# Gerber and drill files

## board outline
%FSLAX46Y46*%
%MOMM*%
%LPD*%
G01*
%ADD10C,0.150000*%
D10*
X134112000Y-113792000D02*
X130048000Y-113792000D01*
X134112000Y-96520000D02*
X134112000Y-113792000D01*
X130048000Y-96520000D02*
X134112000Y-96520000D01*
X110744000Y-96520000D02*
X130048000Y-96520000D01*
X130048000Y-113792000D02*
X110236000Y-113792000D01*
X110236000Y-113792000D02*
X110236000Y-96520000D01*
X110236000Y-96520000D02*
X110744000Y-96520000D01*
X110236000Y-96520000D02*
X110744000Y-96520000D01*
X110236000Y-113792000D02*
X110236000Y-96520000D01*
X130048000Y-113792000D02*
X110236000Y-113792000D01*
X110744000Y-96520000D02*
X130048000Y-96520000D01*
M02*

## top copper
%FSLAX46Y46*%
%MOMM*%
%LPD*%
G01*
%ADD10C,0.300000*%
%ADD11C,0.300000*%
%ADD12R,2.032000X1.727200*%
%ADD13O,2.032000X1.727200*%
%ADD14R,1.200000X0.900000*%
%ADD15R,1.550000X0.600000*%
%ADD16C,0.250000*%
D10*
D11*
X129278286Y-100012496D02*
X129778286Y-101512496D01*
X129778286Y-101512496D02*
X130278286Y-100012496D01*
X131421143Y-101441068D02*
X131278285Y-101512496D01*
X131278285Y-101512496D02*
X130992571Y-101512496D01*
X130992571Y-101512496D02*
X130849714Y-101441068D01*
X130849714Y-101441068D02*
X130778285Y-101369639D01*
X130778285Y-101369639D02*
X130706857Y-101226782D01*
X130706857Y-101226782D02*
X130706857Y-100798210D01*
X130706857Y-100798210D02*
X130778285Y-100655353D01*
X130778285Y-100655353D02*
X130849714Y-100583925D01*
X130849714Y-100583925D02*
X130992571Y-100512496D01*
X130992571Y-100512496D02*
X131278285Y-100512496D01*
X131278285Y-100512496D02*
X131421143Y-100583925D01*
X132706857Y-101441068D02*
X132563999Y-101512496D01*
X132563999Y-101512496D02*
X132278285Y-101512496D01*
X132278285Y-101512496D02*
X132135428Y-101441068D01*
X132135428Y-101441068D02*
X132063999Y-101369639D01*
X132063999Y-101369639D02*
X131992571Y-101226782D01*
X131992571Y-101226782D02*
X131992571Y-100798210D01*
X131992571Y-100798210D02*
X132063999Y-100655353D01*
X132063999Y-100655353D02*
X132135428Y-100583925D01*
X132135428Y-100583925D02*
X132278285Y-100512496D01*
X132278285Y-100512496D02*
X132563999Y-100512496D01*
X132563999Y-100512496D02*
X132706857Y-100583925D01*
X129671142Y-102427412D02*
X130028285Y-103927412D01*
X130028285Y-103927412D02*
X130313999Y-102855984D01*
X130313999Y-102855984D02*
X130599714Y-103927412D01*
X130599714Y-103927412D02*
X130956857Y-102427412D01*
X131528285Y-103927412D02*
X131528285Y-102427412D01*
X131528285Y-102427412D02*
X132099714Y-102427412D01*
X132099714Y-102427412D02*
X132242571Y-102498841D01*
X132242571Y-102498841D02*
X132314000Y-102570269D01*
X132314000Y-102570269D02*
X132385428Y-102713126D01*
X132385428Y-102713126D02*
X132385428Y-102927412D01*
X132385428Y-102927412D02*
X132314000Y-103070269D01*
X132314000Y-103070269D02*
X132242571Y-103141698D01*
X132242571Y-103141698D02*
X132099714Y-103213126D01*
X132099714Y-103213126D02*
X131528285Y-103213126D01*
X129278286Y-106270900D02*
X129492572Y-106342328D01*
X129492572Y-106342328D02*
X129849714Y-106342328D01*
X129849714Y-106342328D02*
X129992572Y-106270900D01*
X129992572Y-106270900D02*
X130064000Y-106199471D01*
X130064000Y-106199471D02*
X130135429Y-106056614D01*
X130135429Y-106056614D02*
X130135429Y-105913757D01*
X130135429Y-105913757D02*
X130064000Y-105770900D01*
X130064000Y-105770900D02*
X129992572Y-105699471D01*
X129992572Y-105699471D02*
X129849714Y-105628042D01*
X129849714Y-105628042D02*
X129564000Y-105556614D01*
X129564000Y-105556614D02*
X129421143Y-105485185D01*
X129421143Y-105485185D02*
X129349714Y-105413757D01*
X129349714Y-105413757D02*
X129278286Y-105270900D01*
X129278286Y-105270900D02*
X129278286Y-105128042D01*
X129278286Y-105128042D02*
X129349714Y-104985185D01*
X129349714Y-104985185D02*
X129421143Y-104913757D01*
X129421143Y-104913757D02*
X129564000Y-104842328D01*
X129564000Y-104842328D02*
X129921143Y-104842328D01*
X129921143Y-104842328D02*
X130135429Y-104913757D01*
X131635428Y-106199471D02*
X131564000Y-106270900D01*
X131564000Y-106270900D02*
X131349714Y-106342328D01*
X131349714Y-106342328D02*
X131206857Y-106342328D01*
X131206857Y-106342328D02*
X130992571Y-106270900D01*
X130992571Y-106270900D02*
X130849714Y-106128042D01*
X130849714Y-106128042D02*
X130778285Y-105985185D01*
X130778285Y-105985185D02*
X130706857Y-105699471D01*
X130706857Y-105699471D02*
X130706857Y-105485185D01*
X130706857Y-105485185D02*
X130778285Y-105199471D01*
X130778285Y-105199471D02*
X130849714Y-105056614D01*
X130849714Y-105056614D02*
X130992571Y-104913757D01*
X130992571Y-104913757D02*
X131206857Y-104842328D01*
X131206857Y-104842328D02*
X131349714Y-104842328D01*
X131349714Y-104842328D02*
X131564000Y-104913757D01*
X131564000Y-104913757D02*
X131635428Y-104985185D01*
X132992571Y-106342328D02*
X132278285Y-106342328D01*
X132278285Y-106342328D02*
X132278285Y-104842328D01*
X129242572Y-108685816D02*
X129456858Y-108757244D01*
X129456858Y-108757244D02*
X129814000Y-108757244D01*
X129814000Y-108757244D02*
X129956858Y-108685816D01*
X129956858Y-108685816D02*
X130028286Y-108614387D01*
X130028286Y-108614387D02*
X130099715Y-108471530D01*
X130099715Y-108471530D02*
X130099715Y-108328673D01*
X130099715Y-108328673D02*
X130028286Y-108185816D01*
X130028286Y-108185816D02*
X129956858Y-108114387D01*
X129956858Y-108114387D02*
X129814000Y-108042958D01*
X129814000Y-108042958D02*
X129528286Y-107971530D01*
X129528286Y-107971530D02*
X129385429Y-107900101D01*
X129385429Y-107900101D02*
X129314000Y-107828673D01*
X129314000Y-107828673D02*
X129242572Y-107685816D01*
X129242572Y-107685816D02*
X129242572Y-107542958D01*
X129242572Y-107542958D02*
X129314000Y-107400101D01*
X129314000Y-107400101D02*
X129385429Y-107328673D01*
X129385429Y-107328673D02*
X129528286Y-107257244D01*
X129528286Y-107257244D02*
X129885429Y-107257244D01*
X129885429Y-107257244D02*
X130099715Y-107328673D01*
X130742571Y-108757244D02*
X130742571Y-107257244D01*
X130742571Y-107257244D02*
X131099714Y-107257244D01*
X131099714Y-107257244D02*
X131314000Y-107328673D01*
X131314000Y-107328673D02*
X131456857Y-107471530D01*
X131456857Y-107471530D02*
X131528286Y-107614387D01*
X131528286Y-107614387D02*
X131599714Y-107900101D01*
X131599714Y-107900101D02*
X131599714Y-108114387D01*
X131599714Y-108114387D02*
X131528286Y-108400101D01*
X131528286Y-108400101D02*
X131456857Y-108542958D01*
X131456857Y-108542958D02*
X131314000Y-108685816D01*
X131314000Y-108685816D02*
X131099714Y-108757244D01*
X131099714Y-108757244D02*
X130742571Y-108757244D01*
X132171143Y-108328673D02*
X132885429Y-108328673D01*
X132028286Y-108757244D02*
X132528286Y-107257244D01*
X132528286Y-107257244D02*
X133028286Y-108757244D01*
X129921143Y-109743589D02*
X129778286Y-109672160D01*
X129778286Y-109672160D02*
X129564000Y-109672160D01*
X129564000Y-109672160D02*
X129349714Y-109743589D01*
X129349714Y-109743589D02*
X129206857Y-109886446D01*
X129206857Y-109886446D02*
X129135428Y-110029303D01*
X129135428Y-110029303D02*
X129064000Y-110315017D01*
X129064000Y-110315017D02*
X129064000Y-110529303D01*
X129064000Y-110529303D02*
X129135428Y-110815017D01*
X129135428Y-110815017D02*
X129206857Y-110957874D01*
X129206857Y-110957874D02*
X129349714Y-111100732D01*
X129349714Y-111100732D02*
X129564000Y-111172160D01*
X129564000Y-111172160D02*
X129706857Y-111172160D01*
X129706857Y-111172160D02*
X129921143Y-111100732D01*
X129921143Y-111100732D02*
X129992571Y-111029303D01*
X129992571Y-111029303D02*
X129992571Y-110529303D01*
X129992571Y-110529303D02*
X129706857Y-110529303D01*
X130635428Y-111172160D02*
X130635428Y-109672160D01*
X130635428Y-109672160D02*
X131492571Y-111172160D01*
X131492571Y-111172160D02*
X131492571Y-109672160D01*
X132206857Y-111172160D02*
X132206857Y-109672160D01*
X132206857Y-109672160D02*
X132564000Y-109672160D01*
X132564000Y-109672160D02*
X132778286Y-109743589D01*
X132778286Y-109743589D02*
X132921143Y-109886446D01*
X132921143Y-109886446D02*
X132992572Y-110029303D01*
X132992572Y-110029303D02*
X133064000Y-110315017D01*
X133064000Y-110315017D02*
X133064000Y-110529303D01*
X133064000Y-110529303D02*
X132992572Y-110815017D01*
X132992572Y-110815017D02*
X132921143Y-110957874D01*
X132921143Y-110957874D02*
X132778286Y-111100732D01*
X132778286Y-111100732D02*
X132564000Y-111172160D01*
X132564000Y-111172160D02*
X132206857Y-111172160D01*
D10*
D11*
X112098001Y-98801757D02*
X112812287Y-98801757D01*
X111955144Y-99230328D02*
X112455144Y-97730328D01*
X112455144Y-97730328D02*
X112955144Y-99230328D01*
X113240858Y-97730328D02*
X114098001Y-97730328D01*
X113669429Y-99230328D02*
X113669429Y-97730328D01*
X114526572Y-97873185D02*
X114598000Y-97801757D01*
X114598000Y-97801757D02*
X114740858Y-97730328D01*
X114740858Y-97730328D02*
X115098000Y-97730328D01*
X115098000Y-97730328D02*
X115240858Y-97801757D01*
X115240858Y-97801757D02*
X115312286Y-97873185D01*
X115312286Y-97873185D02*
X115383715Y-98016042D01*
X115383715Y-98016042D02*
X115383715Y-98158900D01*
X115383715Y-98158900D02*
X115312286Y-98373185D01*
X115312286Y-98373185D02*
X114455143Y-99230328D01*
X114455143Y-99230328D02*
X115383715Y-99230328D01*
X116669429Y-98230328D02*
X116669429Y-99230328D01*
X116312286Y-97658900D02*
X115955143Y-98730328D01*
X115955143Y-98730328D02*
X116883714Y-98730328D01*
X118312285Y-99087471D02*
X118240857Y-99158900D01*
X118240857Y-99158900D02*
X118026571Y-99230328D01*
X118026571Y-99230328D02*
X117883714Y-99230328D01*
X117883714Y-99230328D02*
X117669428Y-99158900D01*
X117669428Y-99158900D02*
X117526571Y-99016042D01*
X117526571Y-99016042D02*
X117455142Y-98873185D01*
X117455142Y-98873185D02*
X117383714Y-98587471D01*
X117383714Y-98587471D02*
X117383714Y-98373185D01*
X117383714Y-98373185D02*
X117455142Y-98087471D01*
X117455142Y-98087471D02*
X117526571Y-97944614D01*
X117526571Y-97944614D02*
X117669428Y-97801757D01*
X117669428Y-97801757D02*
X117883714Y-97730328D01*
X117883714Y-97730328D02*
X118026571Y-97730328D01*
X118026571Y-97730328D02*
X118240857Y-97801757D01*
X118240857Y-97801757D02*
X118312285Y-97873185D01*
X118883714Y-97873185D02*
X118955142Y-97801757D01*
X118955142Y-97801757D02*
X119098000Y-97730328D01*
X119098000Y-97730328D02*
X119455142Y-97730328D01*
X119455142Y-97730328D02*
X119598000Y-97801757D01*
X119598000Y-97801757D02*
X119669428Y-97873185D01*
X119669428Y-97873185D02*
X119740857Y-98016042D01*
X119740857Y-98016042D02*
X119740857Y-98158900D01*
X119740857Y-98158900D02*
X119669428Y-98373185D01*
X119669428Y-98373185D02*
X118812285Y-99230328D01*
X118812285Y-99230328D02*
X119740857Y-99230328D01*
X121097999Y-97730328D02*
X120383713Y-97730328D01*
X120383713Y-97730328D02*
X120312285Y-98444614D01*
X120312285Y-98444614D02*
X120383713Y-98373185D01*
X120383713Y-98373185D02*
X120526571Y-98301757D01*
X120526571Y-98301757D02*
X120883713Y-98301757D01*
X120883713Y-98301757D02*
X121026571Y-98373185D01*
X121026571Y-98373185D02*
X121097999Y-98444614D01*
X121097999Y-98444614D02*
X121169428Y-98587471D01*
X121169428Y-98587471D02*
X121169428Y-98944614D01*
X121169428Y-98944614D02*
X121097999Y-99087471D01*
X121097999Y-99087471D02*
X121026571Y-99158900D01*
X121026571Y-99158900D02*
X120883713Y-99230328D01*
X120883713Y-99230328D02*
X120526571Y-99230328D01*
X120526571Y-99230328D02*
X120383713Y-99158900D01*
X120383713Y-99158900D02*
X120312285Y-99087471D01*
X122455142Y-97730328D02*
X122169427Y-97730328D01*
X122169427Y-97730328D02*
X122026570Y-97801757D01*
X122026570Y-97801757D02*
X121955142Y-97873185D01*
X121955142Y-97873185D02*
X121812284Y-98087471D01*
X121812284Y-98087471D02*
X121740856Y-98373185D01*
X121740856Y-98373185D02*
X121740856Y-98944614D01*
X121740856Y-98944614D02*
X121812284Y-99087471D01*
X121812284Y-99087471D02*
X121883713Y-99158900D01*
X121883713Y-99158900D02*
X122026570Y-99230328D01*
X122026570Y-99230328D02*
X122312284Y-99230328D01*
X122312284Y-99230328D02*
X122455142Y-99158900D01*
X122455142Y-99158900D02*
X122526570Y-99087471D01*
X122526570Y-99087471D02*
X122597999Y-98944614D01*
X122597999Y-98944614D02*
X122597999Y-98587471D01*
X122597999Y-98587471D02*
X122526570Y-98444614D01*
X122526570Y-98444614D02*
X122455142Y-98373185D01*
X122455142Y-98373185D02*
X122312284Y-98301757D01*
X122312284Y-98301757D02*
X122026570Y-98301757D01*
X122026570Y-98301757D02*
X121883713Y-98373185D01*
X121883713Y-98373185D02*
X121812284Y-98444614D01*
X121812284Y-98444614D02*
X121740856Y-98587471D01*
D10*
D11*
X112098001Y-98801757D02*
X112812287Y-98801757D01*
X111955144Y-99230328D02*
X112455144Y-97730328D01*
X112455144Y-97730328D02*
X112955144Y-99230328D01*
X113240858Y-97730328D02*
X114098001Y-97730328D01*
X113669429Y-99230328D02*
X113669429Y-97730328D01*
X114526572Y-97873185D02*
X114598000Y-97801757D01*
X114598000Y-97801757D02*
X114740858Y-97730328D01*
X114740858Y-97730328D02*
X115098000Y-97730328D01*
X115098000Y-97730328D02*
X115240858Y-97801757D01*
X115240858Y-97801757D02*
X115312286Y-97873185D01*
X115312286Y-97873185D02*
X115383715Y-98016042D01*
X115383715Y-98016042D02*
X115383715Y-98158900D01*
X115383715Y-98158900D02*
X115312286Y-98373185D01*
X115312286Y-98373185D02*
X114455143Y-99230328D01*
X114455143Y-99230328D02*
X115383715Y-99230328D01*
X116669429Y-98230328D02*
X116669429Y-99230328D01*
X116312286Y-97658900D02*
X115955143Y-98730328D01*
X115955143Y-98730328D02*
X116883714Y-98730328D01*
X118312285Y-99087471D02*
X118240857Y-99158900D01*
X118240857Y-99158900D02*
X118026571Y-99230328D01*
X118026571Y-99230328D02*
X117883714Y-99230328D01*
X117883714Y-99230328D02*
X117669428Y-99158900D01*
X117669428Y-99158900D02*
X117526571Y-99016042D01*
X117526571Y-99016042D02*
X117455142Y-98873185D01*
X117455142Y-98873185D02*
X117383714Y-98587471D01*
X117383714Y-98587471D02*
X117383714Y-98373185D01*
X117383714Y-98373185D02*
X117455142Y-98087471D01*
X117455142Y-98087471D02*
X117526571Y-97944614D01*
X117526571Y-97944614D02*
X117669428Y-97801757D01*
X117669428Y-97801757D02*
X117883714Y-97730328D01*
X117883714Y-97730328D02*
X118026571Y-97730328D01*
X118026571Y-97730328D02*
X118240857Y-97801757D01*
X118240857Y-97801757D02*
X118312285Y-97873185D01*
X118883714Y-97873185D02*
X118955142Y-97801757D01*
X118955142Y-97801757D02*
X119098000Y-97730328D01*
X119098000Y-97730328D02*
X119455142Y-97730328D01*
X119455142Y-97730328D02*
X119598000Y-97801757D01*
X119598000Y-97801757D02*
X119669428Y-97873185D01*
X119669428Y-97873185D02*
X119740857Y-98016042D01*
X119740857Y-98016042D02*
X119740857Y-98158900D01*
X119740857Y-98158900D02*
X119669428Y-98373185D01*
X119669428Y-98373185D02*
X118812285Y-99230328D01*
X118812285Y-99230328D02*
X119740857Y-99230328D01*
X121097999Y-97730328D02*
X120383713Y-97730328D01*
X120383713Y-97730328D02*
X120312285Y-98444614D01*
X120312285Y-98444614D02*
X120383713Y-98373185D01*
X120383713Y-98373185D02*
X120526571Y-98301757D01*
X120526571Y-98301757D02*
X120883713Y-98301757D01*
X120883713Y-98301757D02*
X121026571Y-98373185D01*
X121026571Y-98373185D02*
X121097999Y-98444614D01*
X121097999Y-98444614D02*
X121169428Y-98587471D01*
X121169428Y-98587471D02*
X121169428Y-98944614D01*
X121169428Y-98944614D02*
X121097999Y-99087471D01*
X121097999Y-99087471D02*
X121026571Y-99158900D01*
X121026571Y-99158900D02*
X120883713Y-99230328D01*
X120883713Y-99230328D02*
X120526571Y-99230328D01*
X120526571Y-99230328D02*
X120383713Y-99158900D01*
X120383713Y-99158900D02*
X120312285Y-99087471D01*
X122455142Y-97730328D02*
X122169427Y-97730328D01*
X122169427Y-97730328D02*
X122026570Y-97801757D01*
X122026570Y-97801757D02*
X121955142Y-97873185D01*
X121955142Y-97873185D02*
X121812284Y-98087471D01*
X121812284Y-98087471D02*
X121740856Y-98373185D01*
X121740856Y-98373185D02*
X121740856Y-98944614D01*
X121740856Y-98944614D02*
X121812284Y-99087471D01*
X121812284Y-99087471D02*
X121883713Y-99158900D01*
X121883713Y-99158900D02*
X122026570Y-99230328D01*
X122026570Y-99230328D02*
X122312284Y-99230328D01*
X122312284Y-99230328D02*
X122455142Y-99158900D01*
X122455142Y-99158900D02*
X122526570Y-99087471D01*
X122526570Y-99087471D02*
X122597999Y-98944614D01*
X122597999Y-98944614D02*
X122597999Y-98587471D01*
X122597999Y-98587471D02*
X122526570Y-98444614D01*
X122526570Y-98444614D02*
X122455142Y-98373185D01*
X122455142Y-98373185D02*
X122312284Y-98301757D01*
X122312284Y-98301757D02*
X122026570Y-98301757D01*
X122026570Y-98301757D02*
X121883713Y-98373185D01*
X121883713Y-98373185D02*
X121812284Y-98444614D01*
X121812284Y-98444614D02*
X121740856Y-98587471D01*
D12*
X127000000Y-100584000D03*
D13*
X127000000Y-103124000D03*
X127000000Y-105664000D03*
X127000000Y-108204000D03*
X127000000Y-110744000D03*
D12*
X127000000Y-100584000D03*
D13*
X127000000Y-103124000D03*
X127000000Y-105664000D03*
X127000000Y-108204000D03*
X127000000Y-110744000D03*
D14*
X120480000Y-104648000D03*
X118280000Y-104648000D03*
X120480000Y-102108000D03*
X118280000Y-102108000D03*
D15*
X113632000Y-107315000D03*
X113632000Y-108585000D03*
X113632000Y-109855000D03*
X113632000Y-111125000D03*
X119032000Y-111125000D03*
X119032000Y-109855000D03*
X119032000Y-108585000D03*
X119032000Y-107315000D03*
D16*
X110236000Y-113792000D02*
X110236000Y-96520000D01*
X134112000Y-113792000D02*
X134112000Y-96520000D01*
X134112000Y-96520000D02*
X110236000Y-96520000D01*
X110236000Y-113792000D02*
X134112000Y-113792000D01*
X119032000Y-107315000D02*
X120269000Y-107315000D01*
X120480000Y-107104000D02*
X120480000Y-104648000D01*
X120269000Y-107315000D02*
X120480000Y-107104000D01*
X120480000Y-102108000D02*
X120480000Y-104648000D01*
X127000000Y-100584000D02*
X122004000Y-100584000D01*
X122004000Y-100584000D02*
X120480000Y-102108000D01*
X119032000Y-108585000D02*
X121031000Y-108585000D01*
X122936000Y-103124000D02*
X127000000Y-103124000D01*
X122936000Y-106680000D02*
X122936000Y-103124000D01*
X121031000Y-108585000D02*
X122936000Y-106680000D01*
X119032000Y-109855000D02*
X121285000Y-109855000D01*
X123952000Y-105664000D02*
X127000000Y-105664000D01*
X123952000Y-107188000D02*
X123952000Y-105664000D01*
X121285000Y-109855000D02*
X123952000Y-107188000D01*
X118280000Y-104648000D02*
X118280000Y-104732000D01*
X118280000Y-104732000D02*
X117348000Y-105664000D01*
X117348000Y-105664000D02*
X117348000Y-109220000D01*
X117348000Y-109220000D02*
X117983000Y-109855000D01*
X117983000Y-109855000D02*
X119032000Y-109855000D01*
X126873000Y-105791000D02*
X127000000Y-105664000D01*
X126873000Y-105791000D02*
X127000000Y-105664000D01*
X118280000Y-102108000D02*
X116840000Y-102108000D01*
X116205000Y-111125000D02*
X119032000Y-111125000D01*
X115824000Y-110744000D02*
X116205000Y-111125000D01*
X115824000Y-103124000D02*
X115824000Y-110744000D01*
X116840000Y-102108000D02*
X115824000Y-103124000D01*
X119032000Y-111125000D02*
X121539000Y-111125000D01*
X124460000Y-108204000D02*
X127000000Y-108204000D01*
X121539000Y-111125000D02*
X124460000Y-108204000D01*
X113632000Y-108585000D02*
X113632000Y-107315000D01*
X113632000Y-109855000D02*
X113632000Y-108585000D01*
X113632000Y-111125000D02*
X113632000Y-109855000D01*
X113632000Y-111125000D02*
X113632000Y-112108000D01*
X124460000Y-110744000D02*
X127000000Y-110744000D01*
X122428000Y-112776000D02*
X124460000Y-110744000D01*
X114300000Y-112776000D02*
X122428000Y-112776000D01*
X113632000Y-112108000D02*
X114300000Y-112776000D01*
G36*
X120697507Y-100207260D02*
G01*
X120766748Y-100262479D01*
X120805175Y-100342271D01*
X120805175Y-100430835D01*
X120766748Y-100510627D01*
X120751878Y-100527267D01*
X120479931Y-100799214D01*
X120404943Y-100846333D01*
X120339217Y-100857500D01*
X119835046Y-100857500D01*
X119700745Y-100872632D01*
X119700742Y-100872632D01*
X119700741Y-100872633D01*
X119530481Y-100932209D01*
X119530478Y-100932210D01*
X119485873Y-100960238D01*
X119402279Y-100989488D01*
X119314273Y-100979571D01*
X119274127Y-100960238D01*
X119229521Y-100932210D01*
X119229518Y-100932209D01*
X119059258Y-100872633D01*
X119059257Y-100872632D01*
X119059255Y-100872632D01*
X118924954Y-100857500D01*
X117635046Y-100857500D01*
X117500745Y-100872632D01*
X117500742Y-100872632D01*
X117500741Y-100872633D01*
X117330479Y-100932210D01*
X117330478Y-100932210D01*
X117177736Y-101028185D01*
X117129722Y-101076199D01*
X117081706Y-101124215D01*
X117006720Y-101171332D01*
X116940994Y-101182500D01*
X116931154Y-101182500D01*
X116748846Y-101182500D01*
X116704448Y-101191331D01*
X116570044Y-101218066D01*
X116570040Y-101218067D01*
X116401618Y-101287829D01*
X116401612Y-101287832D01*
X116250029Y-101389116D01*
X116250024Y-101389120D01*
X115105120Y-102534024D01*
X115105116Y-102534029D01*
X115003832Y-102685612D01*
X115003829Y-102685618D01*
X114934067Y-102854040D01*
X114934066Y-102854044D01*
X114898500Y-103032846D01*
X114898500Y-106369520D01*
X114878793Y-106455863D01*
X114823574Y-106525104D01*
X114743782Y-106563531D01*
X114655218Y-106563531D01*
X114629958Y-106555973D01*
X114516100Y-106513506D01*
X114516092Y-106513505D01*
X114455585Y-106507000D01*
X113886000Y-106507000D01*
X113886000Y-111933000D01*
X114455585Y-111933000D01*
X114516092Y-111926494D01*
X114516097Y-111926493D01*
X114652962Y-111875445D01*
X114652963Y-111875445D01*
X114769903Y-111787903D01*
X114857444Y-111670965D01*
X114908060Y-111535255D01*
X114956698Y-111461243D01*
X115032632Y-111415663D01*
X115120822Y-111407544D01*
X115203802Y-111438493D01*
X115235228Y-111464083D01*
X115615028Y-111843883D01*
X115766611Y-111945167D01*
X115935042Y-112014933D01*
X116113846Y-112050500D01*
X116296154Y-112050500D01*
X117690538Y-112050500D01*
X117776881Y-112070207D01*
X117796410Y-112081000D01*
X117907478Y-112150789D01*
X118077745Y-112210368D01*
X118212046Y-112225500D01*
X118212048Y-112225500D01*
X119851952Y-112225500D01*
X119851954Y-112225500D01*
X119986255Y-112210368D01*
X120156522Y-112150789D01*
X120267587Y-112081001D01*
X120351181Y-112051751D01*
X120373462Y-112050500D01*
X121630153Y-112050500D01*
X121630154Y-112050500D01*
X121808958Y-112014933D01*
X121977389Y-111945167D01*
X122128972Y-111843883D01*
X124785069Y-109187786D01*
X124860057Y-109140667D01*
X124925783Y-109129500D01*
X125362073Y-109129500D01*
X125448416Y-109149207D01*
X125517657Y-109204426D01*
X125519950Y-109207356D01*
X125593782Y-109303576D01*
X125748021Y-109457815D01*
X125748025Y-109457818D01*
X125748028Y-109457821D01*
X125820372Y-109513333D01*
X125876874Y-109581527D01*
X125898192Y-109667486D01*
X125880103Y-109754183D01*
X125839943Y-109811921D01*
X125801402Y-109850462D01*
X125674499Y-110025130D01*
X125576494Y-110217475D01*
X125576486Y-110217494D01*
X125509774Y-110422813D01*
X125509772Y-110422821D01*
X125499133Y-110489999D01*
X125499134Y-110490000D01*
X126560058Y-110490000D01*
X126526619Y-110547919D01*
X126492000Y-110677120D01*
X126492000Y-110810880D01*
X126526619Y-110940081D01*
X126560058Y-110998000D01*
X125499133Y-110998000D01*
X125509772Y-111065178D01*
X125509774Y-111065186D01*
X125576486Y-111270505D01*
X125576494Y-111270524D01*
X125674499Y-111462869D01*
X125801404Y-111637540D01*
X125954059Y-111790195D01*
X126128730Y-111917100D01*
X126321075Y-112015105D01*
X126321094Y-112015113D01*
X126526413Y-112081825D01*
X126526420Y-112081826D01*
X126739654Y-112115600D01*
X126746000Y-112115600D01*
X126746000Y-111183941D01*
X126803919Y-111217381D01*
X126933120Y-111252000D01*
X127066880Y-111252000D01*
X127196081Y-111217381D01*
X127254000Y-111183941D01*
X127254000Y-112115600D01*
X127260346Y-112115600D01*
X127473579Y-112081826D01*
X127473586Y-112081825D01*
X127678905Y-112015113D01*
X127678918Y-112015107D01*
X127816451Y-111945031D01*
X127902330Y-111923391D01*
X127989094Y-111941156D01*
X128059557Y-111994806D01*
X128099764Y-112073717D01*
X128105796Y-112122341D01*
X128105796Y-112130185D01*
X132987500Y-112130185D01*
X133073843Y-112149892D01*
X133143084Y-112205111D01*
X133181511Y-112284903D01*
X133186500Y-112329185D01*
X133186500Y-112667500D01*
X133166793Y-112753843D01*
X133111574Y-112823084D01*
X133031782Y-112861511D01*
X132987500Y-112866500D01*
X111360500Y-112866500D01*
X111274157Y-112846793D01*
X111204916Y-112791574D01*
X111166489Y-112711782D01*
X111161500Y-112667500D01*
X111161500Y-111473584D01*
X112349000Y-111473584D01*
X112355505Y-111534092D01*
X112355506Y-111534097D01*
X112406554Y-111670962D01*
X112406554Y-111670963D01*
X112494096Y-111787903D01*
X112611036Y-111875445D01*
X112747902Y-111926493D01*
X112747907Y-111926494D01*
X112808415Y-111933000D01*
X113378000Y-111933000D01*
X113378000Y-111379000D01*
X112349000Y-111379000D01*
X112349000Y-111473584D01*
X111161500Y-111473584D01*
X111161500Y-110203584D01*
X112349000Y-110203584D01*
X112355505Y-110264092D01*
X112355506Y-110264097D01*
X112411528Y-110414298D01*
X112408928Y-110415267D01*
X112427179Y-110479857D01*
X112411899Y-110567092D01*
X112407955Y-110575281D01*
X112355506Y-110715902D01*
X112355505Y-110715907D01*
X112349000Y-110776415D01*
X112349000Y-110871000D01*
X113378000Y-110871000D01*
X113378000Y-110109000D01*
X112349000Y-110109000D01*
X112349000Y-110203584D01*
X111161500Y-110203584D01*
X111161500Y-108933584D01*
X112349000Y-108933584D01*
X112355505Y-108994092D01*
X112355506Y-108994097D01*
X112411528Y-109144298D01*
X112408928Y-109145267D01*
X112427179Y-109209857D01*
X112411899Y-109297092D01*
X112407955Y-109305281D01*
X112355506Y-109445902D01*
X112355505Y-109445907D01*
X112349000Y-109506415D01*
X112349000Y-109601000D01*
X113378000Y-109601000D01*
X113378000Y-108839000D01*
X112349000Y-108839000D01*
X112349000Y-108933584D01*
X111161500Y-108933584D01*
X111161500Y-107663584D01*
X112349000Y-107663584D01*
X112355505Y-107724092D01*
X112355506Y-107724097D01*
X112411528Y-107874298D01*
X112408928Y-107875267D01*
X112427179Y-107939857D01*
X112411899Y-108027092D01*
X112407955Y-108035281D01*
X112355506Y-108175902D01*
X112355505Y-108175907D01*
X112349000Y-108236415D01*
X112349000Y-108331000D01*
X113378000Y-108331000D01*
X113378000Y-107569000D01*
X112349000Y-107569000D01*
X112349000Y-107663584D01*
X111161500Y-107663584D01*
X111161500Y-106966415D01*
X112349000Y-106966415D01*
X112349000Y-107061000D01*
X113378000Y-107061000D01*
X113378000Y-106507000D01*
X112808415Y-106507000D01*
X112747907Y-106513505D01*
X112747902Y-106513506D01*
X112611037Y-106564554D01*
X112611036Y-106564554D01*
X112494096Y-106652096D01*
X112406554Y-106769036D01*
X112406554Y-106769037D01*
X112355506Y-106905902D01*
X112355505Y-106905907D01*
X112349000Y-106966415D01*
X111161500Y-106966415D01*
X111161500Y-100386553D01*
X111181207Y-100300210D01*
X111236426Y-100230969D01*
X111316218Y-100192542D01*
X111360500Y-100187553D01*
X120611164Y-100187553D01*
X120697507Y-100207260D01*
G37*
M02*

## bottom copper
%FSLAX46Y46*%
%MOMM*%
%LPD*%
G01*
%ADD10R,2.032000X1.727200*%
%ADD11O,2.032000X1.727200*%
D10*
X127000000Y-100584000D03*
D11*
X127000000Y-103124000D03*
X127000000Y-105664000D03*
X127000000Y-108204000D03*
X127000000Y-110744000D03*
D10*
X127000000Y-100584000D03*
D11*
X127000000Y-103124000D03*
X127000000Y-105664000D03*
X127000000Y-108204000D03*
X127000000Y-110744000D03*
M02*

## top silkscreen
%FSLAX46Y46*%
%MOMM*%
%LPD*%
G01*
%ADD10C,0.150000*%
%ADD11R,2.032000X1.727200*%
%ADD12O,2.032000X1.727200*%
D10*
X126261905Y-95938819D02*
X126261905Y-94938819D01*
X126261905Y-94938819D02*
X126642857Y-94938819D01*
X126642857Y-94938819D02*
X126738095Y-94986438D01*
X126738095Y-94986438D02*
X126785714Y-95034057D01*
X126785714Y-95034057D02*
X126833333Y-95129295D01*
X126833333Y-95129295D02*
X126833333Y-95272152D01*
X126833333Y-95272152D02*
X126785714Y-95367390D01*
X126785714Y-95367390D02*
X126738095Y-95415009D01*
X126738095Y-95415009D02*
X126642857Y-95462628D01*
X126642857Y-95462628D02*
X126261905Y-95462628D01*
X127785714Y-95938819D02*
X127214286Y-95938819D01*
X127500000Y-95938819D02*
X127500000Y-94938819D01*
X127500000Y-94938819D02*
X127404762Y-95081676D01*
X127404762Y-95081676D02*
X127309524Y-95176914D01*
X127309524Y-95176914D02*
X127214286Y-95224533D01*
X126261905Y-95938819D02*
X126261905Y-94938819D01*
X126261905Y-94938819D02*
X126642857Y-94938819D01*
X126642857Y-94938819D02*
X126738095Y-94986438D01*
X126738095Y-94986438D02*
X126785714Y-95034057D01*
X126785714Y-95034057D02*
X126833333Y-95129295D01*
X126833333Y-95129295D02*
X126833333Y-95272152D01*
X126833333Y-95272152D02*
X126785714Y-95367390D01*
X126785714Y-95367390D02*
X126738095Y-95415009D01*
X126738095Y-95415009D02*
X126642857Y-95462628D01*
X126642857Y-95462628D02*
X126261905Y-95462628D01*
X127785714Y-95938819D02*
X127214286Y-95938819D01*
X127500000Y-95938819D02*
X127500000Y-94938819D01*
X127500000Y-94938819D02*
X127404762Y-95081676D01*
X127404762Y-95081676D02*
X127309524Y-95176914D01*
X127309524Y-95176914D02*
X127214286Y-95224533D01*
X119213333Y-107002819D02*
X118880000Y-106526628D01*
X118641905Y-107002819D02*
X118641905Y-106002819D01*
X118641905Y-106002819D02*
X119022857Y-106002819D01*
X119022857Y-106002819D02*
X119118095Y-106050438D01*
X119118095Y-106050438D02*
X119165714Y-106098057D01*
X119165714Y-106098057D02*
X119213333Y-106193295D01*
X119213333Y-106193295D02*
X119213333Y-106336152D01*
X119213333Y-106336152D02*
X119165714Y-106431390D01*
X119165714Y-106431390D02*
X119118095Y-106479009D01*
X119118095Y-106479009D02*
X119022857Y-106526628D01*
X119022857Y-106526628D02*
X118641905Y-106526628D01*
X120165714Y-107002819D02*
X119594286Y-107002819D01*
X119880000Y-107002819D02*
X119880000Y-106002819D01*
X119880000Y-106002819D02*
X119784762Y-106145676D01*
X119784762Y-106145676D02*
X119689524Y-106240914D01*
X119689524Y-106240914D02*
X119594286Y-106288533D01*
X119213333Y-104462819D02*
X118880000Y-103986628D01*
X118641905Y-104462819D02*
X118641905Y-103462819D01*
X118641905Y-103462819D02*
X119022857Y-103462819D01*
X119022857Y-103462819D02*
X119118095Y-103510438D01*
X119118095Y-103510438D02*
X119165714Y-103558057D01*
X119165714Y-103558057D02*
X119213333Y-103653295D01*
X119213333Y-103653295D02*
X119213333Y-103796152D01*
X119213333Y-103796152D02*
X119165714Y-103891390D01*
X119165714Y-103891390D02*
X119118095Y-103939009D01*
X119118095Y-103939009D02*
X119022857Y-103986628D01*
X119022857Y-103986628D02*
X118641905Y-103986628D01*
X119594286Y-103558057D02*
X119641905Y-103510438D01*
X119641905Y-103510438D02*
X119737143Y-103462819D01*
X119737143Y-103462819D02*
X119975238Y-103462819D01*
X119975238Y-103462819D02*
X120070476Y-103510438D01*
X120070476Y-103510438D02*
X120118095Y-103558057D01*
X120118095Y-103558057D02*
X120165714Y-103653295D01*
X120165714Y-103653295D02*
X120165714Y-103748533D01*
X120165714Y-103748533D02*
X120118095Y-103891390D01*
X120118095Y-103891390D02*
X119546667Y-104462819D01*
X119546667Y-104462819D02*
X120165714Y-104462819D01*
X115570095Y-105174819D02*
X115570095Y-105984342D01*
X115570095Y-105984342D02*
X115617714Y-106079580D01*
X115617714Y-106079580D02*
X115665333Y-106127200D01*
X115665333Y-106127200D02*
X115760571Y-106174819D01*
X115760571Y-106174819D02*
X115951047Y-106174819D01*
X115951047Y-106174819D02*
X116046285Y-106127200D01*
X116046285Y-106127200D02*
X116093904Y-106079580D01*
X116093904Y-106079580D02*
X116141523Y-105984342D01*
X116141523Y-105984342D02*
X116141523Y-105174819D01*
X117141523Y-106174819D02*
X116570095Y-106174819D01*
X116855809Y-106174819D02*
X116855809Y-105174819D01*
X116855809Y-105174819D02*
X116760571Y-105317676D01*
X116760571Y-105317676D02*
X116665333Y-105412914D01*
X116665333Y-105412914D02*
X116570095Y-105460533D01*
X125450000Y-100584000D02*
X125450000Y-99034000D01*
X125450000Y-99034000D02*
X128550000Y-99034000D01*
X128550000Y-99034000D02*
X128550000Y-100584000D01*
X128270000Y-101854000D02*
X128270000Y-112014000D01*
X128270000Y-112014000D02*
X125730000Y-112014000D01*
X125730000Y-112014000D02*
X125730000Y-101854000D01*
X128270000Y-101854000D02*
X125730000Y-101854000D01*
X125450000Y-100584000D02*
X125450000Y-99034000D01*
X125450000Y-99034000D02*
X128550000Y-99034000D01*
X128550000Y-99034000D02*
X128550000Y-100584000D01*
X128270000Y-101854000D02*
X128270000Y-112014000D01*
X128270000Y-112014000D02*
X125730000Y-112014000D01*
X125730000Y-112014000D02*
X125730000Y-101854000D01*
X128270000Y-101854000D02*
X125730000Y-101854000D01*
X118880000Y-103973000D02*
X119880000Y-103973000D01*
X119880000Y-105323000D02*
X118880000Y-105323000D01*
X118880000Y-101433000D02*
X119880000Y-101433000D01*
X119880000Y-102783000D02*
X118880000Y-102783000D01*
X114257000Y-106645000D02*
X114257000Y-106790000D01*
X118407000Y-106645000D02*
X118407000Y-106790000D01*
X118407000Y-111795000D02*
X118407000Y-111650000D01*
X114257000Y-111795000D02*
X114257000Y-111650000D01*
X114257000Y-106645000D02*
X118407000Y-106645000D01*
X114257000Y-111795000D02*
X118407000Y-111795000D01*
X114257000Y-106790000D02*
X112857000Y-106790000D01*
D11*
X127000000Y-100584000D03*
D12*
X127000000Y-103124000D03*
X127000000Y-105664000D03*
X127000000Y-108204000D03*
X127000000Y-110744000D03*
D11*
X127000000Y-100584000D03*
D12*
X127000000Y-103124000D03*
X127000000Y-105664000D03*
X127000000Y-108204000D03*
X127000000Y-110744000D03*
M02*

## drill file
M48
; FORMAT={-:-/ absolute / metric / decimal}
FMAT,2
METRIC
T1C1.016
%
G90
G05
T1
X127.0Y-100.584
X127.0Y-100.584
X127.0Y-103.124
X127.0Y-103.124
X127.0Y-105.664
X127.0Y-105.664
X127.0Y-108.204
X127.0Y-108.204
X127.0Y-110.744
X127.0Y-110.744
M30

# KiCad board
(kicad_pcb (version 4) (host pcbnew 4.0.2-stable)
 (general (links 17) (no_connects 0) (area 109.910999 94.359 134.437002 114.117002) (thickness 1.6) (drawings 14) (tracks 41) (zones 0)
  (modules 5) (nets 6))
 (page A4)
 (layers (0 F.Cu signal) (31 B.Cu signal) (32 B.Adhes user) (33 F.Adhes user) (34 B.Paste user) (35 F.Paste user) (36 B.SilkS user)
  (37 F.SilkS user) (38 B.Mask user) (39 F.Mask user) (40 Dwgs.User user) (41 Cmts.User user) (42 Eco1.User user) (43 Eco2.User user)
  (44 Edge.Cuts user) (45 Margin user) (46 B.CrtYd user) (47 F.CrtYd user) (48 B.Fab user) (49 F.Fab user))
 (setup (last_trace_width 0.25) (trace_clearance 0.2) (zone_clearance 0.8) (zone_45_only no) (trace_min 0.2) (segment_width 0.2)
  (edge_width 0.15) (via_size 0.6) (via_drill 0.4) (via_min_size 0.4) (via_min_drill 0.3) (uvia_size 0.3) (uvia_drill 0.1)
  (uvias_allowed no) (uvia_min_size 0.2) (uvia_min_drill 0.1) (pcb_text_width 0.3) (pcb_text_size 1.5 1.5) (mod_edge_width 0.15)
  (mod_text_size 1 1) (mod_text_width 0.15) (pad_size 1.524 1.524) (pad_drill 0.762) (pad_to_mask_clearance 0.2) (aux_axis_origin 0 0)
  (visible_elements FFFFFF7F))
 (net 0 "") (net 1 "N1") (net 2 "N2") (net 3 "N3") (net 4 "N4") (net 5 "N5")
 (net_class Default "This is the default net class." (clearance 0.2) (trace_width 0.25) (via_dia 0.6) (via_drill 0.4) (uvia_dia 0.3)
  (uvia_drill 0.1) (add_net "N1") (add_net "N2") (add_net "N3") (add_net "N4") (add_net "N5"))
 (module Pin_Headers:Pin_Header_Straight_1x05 (layer F.Cu) (at 127 100.584)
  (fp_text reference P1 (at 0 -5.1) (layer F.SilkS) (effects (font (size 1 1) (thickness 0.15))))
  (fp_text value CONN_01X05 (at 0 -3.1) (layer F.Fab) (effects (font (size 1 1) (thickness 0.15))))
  (fp_line (start -1.55 0) (end -1.55 -1.55) (layer F.SilkS) (width 0.15))
  (fp_line (start -1.55 -1.55) (end 1.55 -1.55) (layer F.SilkS) (width 0.15))
  (fp_line (start 1.55 -1.55) (end 1.55 0) (layer F.SilkS) (width 0.15))
  (fp_line (start 1.27 1.27) (end 1.27 11.43) (layer F.SilkS) (width 0.15))
  (fp_line (start 1.27 11.43) (end -1.27 11.43) (layer F.SilkS) (width 0.15))
  (fp_line (start -1.27 11.43) (end -1.27 1.27) (layer F.SilkS) (width 0.15))
  (fp_line (start 1.27 1.27) (end -1.27 1.27) (layer F.SilkS) (width 0.15))
  (pad 1 thru_hole rect (at 0 0) (size 2.032 1.7272) (drill 1.016) (layers *.Cu *.Mask F.SilkS) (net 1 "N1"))
  (pad 2 thru_hole oval (at 0 2.54) (size 2.032 1.7272) (drill 1.016) (layers *.Cu *.Mask F.SilkS) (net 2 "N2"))
  (pad 3 thru_hole oval (at 0 5.08) (size 2.032 1.7272) (drill 1.016) (layers *.Cu *.Mask F.SilkS) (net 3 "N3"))
  (pad 4 thru_hole oval (at 0 7.62) (size 2.032 1.7272) (drill 1.016) (layers *.Cu *.Mask F.SilkS) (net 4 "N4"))
  (pad 5 thru_hole oval (at 0 10.16) (size 2.032 1.7272) (drill 1.016) (layers *.Cu *.Mask F.SilkS) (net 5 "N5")))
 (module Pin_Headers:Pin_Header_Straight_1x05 (layer F.Cu) (at 127 100.584)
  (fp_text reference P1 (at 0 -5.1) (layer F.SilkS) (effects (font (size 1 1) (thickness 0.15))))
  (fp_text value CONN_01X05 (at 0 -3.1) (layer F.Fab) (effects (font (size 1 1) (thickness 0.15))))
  (fp_line (start -1.55 0) (end -1.55 -1.55) (layer F.SilkS) (width 0.15))
  (fp_line (start -1.55 -1.55) (end 1.55 -1.55) (layer F.SilkS) (width 0.15))
  (fp_line (start 1.55 -1.55) (end 1.55 0) (layer F.SilkS) (width 0.15))
  (fp_line (start 1.27 1.27) (end 1.27 11.43) (layer F.SilkS) (width 0.15))
  (fp_line (start 1.27 11.43) (end -1.27 11.43) (layer F.SilkS) (width 0.15))
  (fp_line (start -1.27 11.43) (end -1.27 1.27) (layer F.SilkS) (width 0.15))
  (fp_line (start 1.27 1.27) (end -1.27 1.27) (layer F.SilkS) (width 0.15))
  (pad 1 thru_hole rect (at 0 0) (size 2.032 1.7272) (drill 1.016) (layers *.Cu *.Mask F.SilkS) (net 1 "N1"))
  (pad 2 thru_hole oval (at 0 2.54) (size 2.032 1.7272) (drill 1.016) (layers *.Cu *.Mask F.SilkS) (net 2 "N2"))
  (pad 3 thru_hole oval (at 0 5.08) (size 2.032 1.7272) (drill 1.016) (layers *.Cu *.Mask F.SilkS) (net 3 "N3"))
  (pad 4 thru_hole oval (at 0 7.62) (size 2.032 1.7272) (drill 1.016) (layers *.Cu *.Mask F.SilkS) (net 4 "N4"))
  (pad 5 thru_hole oval (at 0 10.16) (size 2.032 1.7272) (drill 1.016) (layers *.Cu *.Mask F.SilkS) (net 5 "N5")))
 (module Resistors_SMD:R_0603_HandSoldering (layer F.Cu) (at 119.38 104.648 180)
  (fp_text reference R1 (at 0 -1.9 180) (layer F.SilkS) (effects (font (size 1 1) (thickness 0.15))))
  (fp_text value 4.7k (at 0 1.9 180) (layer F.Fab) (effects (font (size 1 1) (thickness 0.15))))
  (fp_line (start 0.5 0.675) (end -0.5 0.675) (layer F.SilkS) (width 0.15))
  (fp_line (start -0.5 -0.675) (end 0.5 -0.675) (layer F.SilkS) (width 0.15))
  (pad 1 smd rect (at -1.1 0 180) (size 1.2 0.9) (layers F.Cu F.Paste F.Mask) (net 1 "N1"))
  (pad 2 smd rect (at 1.1 0 180) (size 1.2 0.9) (layers F.Cu F.Paste F.Mask) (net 3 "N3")))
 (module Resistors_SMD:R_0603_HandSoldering (layer F.Cu) (at 119.38 102.108 180)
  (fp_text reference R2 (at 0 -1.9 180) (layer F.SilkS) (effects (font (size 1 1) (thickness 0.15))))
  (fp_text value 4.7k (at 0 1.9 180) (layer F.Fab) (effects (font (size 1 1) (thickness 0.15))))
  (fp_line (start 0.5 0.675) (end -0.5 0.675) (layer F.SilkS) (width 0.15))
  (fp_line (start -0.5 -0.675) (end 0.5 -0.675) (layer F.SilkS) (width 0.15))
  (pad 1 smd rect (at -1.1 0 180) (size 1.2 0.9) (layers F.Cu F.Paste F.Mask) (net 1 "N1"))
  (pad 2 smd rect (at 1.1 0 180) (size 1.2 0.9) (layers F.Cu F.Paste F.Mask) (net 4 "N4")))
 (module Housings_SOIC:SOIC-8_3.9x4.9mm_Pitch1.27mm (layer F.Cu) (at 116.332 109.22)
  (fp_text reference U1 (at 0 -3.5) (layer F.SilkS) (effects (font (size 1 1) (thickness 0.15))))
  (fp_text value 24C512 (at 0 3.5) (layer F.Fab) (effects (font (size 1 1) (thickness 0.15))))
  (fp_line (start -2.075 -2.575) (end -2.075 -2.43) (layer F.SilkS) (width 0.15))
  (fp_line (start 2.075 -2.575) (end 2.075 -2.43) (layer F.SilkS) (width 0.15))
  (fp_line (start 2.075 2.575) (end 2.075 2.43) (layer F.SilkS) (width 0.15))
  (fp_line (start -2.075 2.575) (end -2.075 2.43) (layer F.SilkS) (width 0.15))
  (fp_line (start -2.075 -2.575) (end 2.075 -2.575) (layer F.SilkS) (width 0.15))
  (fp_line (start -2.075 2.575) (end 2.075 2.575) (layer F.SilkS) (width 0.15))
  (fp_line (start -2.075 -2.43) (end -3.475 -2.43) (layer F.SilkS) (width 0.15))
  (pad 1 smd rect (at -2.7 -1.905) (size 1.55 0.6) (layers F.Cu F.Paste F.Mask) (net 5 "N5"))
  (pad 2 smd rect (at -2.7 -0.635) (size 1.55 0.6) (layers F.Cu F.Paste F.Mask) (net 5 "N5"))
  (pad 3 smd rect (at -2.7 0.635) (size 1.55 0.6) (layers F.Cu F.Paste F.Mask) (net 5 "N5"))
  (pad 4 smd rect (at -2.7 1.905) (size 1.55 0.6) (layers F.Cu F.Paste F.Mask) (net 5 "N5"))
  (pad 5 smd rect (at 2.7 1.905) (size 1.55 0.6) (layers F.Cu F.Paste F.Mask) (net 4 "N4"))
  (pad 6 smd rect (at 2.7 0.635) (size 1.55 0.6) (layers F.Cu F.Paste F.Mask) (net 3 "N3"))
  (pad 7 smd rect (at 2.7 -0.635) (size 1.55 0.6) (layers F.Cu F.Paste F.Mask) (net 2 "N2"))
  (pad 8 smd rect (at 2.7 -1.905) (size 1.55 0.6) (layers F.Cu F.Paste F.Mask) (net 1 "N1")))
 (gr_line (start 134.112 113.792) (end 130.048 113.792) (angle 90) (layer Edge.Cuts) (width 0.15))
 (gr_line (start 134.112 96.52) (end 134.112 113.792) (angle 90) (layer Edge.Cuts) (width 0.15))
 (gr_line (start 130.048 96.52) (end 134.112 96.52) (angle 90) (layer Edge.Cuts) (width 0.15))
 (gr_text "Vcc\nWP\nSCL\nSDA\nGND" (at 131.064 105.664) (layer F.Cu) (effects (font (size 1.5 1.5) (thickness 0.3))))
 (gr_line (start 110.744 96.52) (end 130.048 96.52) (angle 90) (layer Edge.Cuts) (width 0.15))
 (gr_line (start 130.048 113.792) (end 110.236 113.792) (angle 90) (layer Edge.Cuts) (width 0.15))
 (gr_line (start 110.236 113.792) (end 110.236 96.52) (angle 90) (layer Edge.Cuts) (width 0.15))
 (gr_line (start 110.236 96.52) (end 110.744 96.52) (angle 90) (layer Edge.Cuts) (width 0.15))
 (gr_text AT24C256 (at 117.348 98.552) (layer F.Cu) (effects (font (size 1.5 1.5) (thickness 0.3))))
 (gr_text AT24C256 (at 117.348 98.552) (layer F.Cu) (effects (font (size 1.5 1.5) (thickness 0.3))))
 (gr_line (start 110.236 96.52) (end 110.744 96.52) (angle 90) (layer Edge.Cuts) (width 0.15))
 (gr_line (start 110.236 113.792) (end 110.236 96.52) (angle 90) (layer Edge.Cuts) (width 0.15))
 (gr_line (start 130.048 113.792) (end 110.236 113.792) (angle 90) (layer Edge.Cuts) (width 0.15))
 (gr_line (start 110.744 96.52) (end 130.048 96.52) (angle 90) (layer Edge.Cuts) (width 0.15))
 (segment (start 110.236 113.792) (end 110.236 96.52) (width 0.25) (layer F.Cu) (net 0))
 (segment (start 134.112 113.792) (end 134.112 96.52) (width 0.25) (layer F.Cu) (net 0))
 (segment (start 134.112 96.52) (end 110.236 96.52) (width 0.25) (layer F.Cu) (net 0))
 (segment (start 110.236 113.792) (end 134.112 113.792) (width 0.25) (layer F.Cu) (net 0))
 (segment (start 119.032 107.315) (end 120.269 107.315) (width 0.25) (layer F.Cu) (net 1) (status 400000))
 (segment (start 120.48 107.104) (end 120.48 104.648) (width 0.25) (layer F.Cu) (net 1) (status 800000))
 (segment (start 120.269 107.315) (end 120.48 107.104) (width 0.25) (layer F.Cu) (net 1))
 (segment (start 120.48 102.108) (end 120.48 104.648) (width 0.25) (layer F.Cu) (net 1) (status C00000))
 (segment (start 127 100.584) (end 122.004 100.584) (width 0.25) (layer F.Cu) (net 1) (status 400000))
 (segment (start 122.004 100.584) (end 120.48 102.108) (width 0.25) (layer F.Cu) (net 1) (status 800000))
 (segment (start 119.032 108.585) (end 121.031 108.585) (width 0.25) (layer F.Cu) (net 2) (status 400000))
 (segment (start 122.936 103.124) (end 127 103.124) (width 0.25) (layer F.Cu) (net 2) (status 800000))
 (segment (start 122.936 106.68) (end 122.936 103.124) (width 0.25) (layer F.Cu) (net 2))
 (segment (start 121.031 108.585) (end 122.936 106.68) (width 0.25) (layer F.Cu) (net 2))
 (segment (start 119.032 109.855) (end 121.285 109.855) (width 0.25) (layer F.Cu) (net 3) (status 400000))
 (segment (start 123.952 105.664) (end 127 105.664) (width 0.25) (layer F.Cu) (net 3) (status 800000))
 (segment (start 123.952 107.188) (end 123.952 105.664) (width 0.25) (layer F.Cu) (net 3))
 (segment (start 121.285 109.855) (end 123.952 107.188) (width 0.25) (layer F.Cu) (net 3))
 (segment (start 118.28 104.648) (end 118.28 104.732) (width 0.25) (layer F.Cu) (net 3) (status C00000))
 (segment (start 118.28 104.732) (end 117.348 105.664) (width 0.25) (layer F.Cu) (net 3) (status 400000))
 (segment (start 117.348 105.664) (end 117.348 109.22) (width 0.25) (layer F.Cu) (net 3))
 (segment (start 117.348 109.22) (end 117.983 109.855) (width 0.25) (layer F.Cu) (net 3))
 (segment (start 117.983 109.855) (end 119.032 109.855) (width 0.25) (layer F.Cu) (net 3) (status 800000))
 (segment (start 126.873 105.791) (end 127 105.664) (width 0.25) (layer F.Cu) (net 3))
 (segment (start 126.873 105.791) (end 127 105.664) (width 0.25) (layer F.Cu) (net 3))
 (segment (start 118.28 102.108) (end 116.84 102.108) (width 0.25) (layer F.Cu) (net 4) (status 400000))
 (segment (start 116.205 111.125) (end 119.032 111.125) (width 0.25) (layer F.Cu) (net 4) (status 800000))
 (segment (start 115.824 110.744) (end 116.205 111.125) (width 0.25) (layer F.Cu) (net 4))
 (segment (start 115.824 103.124) (end 115.824 110.744) (width 0.25) (layer F.Cu) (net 4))
 (segment (start 116.84 102.108) (end 115.824 103.124) (width 0.25) (layer F.Cu) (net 4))
 (segment (start 119.032 111.125) (end 121.539 111.125) (width 0.25) (layer F.Cu) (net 4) (status 400000))
 (segment (start 124.46 108.204) (end 127 108.204) (width 0.25) (layer F.Cu) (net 4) (status 800000))
 (segment (start 121.539 111.125) (end 124.46 108.204) (width 0.25) (layer F.Cu) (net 4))
 (segment (start 113.632 108.585) (end 113.632 107.315) (width 0.25) (layer F.Cu) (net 5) (status C00000))
 (segment (start 113.632 109.855) (end 113.632 108.585) (width 0.25) (layer F.Cu) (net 5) (status C00000))
 (segment (start 113.632 111.125) (end 113.632 109.855) (width 0.25) (layer F.Cu) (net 5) (status C00000))
 (segment (start 113.632 111.125) (end 113.632 112.108) (width 0.25) (layer F.Cu) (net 5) (status 400000))
 (segment (start 124.46 110.744) (end 127 110.744) (width 0.25) (layer F.Cu) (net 5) (status 800000))
 (segment (start 122.428 112.776) (end 124.46 110.744) (width 0.25) (layer F.Cu) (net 5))
 (segment (start 114.3 112.776) (end 122.428 112.776) (width 0.25) (layer F.Cu) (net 5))
 (segment (start 113.632 112.108) (end 114.3 112.776) (width 0.25) (layer F.Cu) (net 5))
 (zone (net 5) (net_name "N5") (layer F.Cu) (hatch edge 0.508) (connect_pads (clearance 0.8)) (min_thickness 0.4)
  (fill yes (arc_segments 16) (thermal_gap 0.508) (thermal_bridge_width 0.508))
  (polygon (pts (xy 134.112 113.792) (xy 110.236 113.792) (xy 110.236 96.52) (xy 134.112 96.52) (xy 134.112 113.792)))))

